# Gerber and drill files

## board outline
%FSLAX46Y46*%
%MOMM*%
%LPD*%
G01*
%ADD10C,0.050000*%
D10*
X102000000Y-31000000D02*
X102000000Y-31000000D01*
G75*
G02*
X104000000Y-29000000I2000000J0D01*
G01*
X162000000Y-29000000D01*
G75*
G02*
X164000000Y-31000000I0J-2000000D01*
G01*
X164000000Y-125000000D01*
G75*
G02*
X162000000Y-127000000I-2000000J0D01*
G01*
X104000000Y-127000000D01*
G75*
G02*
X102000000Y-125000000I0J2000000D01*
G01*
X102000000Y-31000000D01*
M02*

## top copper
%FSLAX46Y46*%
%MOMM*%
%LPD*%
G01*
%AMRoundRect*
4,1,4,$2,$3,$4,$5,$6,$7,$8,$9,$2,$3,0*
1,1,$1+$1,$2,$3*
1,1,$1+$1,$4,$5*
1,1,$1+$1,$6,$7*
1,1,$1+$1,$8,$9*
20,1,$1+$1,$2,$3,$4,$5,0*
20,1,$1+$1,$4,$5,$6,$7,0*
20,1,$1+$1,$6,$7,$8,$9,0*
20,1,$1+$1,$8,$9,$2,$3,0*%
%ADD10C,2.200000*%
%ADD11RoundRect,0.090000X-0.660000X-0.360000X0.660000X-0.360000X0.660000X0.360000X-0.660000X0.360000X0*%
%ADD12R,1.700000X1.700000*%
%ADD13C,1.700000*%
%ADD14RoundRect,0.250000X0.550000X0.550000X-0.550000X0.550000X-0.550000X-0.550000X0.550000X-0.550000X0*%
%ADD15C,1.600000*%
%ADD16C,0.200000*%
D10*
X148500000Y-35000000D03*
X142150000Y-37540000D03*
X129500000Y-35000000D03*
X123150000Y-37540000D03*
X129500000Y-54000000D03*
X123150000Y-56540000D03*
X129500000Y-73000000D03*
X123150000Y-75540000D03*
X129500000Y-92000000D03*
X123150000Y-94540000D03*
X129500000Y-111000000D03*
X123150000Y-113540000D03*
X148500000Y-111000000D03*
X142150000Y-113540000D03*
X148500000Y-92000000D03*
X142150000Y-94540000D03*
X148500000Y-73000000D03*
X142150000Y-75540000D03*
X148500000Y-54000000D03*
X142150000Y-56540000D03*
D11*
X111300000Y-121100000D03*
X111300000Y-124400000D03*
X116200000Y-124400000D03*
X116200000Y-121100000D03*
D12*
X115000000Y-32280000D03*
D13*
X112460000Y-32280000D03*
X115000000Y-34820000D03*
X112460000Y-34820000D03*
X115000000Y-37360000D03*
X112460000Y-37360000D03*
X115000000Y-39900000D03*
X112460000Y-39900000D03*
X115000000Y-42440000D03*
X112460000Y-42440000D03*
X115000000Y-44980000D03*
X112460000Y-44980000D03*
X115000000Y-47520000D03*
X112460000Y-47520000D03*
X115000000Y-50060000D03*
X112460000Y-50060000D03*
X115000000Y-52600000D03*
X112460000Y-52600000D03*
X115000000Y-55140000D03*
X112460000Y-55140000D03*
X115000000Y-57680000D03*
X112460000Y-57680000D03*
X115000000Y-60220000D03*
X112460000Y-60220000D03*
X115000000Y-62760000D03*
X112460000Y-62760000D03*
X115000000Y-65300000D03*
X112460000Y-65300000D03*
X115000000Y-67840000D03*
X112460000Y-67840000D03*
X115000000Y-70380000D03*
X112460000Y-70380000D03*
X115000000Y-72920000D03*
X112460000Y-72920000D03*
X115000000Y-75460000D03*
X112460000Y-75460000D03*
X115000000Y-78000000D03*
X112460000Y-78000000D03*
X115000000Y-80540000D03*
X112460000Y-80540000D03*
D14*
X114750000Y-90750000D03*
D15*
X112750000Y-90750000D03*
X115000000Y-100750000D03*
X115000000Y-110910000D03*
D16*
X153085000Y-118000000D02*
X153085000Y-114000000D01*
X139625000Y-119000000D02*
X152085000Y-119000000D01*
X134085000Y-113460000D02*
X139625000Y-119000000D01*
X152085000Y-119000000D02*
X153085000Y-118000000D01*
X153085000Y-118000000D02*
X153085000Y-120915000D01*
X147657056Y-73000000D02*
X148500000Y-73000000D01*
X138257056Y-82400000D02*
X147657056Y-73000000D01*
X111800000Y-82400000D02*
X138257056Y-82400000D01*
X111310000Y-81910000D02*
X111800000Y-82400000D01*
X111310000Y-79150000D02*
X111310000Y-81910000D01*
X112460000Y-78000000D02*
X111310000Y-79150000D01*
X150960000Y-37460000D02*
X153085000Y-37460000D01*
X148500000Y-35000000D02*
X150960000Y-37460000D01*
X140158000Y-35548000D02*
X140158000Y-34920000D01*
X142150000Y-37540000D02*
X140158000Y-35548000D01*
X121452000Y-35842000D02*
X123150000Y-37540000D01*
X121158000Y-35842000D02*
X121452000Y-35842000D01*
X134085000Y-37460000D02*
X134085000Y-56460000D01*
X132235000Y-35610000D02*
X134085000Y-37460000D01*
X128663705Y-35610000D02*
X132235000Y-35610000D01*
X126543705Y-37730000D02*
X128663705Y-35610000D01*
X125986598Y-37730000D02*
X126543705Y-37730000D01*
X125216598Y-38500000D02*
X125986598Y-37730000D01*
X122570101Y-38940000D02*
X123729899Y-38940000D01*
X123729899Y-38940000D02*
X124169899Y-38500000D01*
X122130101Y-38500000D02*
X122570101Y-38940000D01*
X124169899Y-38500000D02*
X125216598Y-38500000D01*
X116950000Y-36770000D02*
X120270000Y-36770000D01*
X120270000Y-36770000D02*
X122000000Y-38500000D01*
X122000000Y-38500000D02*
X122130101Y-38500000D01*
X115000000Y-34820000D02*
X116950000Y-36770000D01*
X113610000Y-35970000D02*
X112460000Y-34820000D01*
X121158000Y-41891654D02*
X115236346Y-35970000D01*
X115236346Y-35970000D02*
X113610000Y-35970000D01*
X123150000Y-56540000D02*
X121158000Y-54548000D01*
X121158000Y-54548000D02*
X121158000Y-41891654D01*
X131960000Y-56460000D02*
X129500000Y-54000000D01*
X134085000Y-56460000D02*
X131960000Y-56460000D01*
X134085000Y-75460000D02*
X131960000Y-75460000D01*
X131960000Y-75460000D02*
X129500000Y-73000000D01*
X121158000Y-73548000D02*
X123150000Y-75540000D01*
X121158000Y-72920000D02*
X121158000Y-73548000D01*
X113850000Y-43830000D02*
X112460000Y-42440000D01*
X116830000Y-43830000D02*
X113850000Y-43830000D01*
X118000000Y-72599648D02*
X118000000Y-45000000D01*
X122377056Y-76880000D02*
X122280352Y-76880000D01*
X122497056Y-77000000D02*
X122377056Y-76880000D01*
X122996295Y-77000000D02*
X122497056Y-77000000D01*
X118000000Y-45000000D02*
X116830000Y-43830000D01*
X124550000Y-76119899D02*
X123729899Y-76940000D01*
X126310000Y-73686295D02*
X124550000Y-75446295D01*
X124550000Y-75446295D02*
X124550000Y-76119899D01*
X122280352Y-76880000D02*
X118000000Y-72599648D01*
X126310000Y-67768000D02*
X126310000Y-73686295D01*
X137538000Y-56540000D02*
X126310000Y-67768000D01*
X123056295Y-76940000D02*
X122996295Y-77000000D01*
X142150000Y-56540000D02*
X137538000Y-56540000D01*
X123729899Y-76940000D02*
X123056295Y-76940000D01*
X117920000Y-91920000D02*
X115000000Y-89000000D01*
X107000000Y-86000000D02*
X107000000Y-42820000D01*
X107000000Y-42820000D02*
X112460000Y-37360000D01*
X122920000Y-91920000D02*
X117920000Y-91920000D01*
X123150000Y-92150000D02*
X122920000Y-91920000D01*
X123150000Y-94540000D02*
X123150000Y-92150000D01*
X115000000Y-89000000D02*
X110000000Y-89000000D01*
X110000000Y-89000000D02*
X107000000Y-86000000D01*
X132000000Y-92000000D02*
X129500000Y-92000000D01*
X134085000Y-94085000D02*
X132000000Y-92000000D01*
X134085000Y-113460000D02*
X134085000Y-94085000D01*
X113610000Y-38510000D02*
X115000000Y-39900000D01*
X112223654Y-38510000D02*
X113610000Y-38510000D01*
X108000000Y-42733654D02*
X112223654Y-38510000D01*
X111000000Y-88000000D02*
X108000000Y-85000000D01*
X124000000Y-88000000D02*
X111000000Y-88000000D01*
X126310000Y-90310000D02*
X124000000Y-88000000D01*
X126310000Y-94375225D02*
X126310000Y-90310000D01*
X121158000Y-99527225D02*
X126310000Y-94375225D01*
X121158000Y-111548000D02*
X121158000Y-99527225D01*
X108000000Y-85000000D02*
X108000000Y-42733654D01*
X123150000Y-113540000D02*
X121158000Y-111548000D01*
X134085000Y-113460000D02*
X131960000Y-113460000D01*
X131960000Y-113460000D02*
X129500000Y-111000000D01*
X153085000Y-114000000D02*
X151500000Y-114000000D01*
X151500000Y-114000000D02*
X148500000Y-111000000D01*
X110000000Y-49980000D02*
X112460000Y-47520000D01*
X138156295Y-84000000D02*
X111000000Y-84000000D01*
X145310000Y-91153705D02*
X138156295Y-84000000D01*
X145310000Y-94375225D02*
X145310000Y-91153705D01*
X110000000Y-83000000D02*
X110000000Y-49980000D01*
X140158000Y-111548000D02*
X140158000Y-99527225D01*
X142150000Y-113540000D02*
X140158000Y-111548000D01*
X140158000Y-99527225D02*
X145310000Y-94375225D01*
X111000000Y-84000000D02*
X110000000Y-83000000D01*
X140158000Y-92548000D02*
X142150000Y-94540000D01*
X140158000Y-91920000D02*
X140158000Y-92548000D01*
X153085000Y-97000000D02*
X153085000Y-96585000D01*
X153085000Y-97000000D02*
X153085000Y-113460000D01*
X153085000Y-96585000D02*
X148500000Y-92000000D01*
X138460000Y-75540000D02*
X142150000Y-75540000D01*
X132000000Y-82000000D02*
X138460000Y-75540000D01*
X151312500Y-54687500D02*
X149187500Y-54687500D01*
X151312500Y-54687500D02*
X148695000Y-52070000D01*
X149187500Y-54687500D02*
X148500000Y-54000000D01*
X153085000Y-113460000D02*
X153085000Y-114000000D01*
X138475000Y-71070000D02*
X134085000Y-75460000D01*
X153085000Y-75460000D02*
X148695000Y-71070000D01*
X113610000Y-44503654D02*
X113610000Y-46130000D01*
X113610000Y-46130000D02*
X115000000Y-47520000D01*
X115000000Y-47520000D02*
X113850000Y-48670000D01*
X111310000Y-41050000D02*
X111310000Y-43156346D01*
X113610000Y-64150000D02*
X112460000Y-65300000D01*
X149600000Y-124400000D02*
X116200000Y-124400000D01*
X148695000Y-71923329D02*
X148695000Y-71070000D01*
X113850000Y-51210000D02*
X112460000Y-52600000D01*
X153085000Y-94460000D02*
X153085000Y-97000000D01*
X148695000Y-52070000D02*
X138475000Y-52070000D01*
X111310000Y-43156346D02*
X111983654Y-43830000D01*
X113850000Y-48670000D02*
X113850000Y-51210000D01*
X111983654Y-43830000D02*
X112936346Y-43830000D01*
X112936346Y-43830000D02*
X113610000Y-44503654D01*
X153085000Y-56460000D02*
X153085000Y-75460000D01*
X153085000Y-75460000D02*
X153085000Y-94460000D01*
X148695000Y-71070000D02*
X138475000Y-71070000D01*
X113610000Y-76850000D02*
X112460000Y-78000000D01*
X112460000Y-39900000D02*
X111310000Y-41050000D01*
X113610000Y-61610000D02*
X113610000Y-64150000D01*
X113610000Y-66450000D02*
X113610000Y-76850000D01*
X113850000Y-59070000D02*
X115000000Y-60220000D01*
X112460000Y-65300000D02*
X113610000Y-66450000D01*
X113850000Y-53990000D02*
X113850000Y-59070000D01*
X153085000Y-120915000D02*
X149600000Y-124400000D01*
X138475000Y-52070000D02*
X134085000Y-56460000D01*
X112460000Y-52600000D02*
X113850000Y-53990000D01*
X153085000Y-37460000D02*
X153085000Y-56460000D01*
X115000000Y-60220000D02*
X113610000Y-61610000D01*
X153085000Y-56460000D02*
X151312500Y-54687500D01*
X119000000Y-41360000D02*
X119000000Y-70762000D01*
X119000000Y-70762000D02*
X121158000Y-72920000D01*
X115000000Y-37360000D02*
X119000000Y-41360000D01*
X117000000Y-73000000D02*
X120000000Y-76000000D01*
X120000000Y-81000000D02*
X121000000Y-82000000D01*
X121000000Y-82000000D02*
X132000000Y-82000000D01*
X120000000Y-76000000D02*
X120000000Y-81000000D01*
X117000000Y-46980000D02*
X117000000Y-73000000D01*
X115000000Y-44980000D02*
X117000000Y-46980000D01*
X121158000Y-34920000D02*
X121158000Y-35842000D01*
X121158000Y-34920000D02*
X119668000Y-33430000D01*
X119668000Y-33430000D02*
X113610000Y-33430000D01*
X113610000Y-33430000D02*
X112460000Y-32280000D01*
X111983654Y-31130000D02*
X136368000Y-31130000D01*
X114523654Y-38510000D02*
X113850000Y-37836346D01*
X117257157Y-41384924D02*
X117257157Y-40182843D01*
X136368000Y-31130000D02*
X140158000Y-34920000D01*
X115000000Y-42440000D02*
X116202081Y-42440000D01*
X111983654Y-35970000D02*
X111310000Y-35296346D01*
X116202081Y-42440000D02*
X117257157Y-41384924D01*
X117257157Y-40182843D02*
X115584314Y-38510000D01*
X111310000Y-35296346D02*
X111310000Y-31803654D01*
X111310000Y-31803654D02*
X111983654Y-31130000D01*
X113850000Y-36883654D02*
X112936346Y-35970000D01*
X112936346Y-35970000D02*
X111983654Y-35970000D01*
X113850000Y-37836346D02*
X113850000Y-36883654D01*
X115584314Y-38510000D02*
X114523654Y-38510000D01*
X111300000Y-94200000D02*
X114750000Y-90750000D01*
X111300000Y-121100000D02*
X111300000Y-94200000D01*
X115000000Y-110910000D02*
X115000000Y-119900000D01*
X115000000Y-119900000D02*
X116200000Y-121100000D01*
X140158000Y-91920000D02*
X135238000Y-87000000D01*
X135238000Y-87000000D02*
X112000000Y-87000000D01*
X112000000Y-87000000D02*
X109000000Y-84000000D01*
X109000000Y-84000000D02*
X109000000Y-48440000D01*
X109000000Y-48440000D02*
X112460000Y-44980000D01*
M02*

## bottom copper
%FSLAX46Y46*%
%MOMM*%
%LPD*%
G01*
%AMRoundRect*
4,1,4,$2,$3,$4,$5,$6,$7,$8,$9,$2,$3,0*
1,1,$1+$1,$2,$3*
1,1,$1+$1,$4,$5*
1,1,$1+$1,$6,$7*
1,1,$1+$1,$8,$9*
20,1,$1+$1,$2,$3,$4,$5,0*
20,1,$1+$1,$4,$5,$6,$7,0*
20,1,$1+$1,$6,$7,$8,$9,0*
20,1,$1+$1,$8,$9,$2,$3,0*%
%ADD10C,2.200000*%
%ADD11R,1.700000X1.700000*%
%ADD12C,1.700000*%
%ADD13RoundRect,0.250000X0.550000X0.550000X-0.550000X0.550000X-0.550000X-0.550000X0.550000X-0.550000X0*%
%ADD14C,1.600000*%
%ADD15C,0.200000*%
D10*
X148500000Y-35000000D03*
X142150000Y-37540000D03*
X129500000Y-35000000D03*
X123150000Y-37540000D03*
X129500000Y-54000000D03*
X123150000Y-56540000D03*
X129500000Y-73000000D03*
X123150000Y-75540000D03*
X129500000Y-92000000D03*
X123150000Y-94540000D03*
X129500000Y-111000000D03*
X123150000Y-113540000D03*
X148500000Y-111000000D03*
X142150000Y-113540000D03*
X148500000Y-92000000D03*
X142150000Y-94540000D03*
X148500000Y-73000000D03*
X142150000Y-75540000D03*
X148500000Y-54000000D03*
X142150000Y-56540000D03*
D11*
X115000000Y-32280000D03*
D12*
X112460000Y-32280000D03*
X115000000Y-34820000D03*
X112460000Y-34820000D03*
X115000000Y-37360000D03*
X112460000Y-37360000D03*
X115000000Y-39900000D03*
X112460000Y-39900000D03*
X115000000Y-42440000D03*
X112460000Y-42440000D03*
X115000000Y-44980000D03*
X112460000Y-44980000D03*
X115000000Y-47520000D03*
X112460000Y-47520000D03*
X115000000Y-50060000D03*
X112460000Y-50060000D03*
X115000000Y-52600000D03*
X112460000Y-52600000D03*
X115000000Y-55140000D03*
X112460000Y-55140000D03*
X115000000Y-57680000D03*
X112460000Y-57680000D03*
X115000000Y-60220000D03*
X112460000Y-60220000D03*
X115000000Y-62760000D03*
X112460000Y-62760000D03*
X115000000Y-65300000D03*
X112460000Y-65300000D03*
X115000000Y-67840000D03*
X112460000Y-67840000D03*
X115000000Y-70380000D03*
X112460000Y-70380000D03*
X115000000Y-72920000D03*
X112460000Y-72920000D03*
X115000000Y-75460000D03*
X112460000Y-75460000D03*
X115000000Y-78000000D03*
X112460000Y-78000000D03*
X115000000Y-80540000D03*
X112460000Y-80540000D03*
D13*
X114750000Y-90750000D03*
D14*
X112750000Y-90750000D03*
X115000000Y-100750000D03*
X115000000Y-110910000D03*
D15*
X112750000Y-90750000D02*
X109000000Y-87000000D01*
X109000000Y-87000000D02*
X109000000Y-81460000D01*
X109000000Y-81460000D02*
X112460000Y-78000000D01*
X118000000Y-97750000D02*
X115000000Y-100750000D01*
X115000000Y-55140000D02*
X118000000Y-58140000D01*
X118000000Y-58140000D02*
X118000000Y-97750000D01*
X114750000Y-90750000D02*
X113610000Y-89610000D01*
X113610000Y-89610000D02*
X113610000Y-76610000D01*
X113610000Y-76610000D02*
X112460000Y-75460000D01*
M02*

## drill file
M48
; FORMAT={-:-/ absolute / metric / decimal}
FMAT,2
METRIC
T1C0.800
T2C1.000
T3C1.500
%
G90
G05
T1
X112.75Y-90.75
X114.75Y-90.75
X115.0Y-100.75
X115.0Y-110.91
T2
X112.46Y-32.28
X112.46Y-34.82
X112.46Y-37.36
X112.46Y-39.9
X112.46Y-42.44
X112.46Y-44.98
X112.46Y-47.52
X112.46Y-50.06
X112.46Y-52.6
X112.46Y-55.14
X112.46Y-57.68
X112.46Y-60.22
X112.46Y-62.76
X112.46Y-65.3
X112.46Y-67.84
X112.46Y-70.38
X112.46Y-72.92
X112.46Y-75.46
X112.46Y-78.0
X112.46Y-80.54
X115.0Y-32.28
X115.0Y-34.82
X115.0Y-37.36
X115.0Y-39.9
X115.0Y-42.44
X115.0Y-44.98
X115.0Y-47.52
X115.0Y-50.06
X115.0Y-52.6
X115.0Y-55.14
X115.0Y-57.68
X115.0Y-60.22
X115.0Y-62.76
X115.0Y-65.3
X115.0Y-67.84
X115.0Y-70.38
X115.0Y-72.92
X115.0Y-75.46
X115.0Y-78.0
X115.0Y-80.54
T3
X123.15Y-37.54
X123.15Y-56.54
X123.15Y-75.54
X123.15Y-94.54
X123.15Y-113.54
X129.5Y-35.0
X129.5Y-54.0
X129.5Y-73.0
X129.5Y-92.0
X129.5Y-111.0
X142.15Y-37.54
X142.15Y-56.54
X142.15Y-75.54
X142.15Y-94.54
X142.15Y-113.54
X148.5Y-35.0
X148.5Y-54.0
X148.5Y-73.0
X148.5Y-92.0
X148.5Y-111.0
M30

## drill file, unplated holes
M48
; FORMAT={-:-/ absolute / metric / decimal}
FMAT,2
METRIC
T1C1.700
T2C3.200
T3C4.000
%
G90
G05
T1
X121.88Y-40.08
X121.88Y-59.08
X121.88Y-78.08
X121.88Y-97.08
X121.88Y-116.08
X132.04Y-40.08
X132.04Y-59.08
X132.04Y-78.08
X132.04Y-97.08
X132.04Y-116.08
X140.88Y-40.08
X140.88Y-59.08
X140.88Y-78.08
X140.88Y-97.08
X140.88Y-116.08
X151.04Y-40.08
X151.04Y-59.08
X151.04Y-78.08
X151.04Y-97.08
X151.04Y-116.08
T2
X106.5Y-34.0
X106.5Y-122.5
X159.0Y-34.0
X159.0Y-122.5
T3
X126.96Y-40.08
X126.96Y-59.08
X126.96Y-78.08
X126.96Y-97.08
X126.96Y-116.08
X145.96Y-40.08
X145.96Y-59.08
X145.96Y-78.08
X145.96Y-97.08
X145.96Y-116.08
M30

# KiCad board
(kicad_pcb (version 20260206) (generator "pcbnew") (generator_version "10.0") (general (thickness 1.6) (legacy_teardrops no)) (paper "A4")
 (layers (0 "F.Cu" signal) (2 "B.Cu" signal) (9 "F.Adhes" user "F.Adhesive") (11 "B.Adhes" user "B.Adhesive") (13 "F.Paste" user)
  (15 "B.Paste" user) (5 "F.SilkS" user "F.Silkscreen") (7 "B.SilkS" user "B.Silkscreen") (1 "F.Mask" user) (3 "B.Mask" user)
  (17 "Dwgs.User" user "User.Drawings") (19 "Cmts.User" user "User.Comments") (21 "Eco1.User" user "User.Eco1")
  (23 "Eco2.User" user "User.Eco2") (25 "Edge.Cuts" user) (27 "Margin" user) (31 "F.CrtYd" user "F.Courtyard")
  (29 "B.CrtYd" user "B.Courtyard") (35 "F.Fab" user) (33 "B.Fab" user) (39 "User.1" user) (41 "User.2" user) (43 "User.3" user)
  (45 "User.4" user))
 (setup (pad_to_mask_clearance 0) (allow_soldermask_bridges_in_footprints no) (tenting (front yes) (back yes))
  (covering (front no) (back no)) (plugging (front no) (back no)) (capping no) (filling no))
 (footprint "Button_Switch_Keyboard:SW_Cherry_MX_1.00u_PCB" (layer "F.Cu") (at 148.5 35)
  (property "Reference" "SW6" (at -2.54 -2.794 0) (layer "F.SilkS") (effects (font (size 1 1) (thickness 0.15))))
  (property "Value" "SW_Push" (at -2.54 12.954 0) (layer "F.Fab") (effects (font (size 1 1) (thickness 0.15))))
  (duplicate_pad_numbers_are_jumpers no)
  (pad "" np_thru_hole circle (at -7.62 5.08) (size 1.7 1.7) (drill 1.7) (layers "*.Cu" "*.Mask"))
  (pad "" np_thru_hole circle (at -2.54 5.08) (size 4 4) (drill 4) (layers "*.Cu" "*.Mask"))
  (pad "" np_thru_hole circle (at 2.54 5.08) (size 1.7 1.7) (drill 1.7) (layers "*.Cu" "*.Mask"))
  (pad "1" thru_hole circle (at 0 0) (size 2.2 2.2) (drill 1.5) (layers "*.Cu" "*.Mask") (remove_unused_layers no) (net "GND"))
  (pad "2" thru_hole circle (at -6.35 2.54) (size 2.2 2.2) (drill 1.5) (layers "*.Cu" "*.Mask") (remove_unused_layers no)
   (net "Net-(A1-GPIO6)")))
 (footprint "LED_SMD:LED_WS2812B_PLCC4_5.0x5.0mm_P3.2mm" (layer "F.Cu") (at 113.75 122.75)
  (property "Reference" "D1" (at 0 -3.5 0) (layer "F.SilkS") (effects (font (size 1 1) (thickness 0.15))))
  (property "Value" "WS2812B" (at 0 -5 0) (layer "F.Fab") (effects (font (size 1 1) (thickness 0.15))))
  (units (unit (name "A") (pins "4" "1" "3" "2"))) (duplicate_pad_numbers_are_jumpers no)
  (pad "1" smd roundrect (at -2.45 -1.65) (size 1.5 0.9) (layers "F.Cu" "F.Mask" "F.Paste") (roundrect_rratio 0.1) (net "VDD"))
  (pad "2" smd roundrect (at -2.45 1.65) (size 1.5 0.9) (layers "F.Cu" "F.Mask" "F.Paste") (roundrect_rratio 0.1)
   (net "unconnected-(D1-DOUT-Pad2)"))
  (pad "3" smd roundrect (at 2.45 1.65) (size 1.5 0.9) (layers "F.Cu" "F.Mask" "F.Paste") (roundrect_rratio 0.1) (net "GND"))
  (pad "4" smd roundrect (at 2.45 -1.65) (size 1.5 0.9) (layers "F.Cu" "F.Mask" "F.Paste") (roundrect_rratio 0.1) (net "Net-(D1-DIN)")))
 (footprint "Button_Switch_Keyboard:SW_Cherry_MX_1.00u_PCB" (layer "F.Cu") (at 129.5 73)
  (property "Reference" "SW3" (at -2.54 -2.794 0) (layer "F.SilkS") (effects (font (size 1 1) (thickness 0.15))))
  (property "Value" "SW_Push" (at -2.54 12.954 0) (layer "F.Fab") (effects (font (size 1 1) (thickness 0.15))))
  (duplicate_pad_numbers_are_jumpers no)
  (pad "" np_thru_hole circle (at -7.62 5.08) (size 1.7 1.7) (drill 1.7) (layers "*.Cu" "*.Mask"))
  (pad "" np_thru_hole circle (at -2.54 5.08) (size 4 4) (drill 4) (layers "*.Cu" "*.Mask"))
  (pad "" np_thru_hole circle (at 2.54 5.08) (size 1.7 1.7) (drill 1.7) (layers "*.Cu" "*.Mask"))
  (pad "1" thru_hole circle (at 0 0) (size 2.2 2.2) (drill 1.5) (layers "*.Cu" "*.Mask") (remove_unused_layers no) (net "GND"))
  (pad "2" thru_hole circle (at -6.35 2.54) (size 2.2 2.2) (drill 1.5) (layers "*.Cu" "*.Mask") (remove_unused_layers no)
   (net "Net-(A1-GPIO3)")))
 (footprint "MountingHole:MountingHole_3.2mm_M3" (layer "F.Cu") (at 159 34)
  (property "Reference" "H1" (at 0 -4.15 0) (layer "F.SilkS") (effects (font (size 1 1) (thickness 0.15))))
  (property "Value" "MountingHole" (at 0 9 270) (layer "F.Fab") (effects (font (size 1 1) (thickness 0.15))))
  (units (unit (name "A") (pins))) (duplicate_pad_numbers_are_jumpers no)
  (pad "" np_thru_hole circle (at 0 0) (size 3.2 3.2) (drill 3.2) (layers "*.Cu" "*.Mask")))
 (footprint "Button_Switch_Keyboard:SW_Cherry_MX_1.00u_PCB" (layer "F.Cu") (at 129.5 35)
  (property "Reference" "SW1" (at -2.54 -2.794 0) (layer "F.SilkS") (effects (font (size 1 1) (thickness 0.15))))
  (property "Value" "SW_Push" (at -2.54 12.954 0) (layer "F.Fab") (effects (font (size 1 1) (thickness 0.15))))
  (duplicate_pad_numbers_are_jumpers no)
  (pad "" np_thru_hole circle (at -7.62 5.08) (size 1.7 1.7) (drill 1.7) (layers "*.Cu" "*.Mask"))
  (pad "" np_thru_hole circle (at -2.54 5.08) (size 4 4) (drill 4) (layers "*.Cu" "*.Mask"))
  (pad "" np_thru_hole circle (at 2.54 5.08) (size 1.7 1.7) (drill 1.7) (layers "*.Cu" "*.Mask"))
  (pad "1" thru_hole circle (at 0 0) (size 2.2 2.2) (drill 1.5) (layers "*.Cu" "*.Mask") (remove_unused_layers no) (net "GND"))
  (pad "2" thru_hole circle (at -6.35 2.54) (size 2.2 2.2) (drill 1.5) (layers "*.Cu" "*.Mask") (remove_unused_layers no)
   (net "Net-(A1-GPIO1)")))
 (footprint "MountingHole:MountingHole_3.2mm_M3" (layer "F.Cu") (at 159 122.5)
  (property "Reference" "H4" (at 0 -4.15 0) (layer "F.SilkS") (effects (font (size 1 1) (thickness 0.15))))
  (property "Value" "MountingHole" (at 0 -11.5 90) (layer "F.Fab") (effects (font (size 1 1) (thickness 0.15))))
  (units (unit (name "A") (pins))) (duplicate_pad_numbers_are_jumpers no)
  (pad "" np_thru_hole circle (at 0 0) (size 3.2 3.2) (drill 3.2) (layers "*.Cu" "*.Mask")))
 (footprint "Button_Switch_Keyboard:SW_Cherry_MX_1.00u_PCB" (layer "F.Cu") (at 148.5 92)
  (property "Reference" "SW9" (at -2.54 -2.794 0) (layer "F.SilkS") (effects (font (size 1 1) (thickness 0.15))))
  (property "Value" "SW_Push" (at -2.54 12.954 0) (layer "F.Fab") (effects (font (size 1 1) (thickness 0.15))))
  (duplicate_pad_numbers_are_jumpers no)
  (pad "" np_thru_hole circle (at -7.62 5.08) (size 1.7 1.7) (drill 1.7) (layers "*.Cu" "*.Mask"))
  (pad "" np_thru_hole circle (at -2.54 5.08) (size 4 4) (drill 4) (layers "*.Cu" "*.Mask"))
  (pad "" np_thru_hole circle (at 2.54 5.08) (size 1.7 1.7) (drill 1.7) (layers "*.Cu" "*.Mask"))
  (pad "1" thru_hole circle (at 0 0) (size 2.2 2.2) (drill 1.5) (layers "*.Cu" "*.Mask") (remove_unused_layers no) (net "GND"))
  (pad "2" thru_hole circle (at -6.35 2.54) (size 2.2 2.2) (drill 1.5) (layers "*.Cu" "*.Mask") (remove_unused_layers no)
   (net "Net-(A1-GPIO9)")))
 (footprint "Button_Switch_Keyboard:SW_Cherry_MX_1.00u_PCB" (layer "F.Cu") (at 148.5 54)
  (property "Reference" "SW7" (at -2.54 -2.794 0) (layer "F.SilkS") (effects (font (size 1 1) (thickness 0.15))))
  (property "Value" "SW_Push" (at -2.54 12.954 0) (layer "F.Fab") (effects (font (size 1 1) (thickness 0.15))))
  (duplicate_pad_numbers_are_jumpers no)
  (pad "" np_thru_hole circle (at -7.62 5.08) (size 1.7 1.7) (drill 1.7) (layers "*.Cu" "*.Mask"))
  (pad "" np_thru_hole circle (at -2.54 5.08) (size 4 4) (drill 4) (layers "*.Cu" "*.Mask"))
  (pad "" np_thru_hole circle (at 2.54 5.08) (size 1.7 1.7) (drill 1.7) (layers "*.Cu" "*.Mask"))
  (pad "1" thru_hole circle (at 0 0) (size 2.2 2.2) (drill 1.5) (layers "*.Cu" "*.Mask") (remove_unused_layers no) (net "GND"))
  (pad "2" thru_hole circle (at -6.35 2.54) (size 2.2 2.2) (drill 1.5) (layers "*.Cu" "*.Mask") (remove_unused_layers no)
   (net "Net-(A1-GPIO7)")))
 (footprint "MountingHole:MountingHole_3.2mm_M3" (layer "F.Cu") (at 106.5 34)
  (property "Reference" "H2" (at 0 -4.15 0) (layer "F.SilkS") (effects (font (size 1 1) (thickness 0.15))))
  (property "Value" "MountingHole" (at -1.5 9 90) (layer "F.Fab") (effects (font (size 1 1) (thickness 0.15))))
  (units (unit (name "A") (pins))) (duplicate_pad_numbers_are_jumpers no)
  (pad "" np_thru_hole circle (at 0 0) (size 3.2 3.2) (drill 3.2) (layers "*.Cu" "*.Mask")))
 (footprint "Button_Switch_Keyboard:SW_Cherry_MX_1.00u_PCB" (layer "F.Cu") (at 148.5 111)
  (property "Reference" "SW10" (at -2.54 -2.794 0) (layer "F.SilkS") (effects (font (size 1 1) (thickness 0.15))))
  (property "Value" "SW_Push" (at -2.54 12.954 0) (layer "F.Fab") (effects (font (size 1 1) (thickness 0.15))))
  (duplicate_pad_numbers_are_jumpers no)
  (pad "" np_thru_hole circle (at -7.62 5.08) (size 1.7 1.7) (drill 1.7) (layers "*.Cu" "*.Mask"))
  (pad "" np_thru_hole circle (at -2.54 5.08) (size 4 4) (drill 4) (layers "*.Cu" "*.Mask"))
  (pad "" np_thru_hole circle (at 2.54 5.08) (size 1.7 1.7) (drill 1.7) (layers "*.Cu" "*.Mask"))
  (pad "1" thru_hole circle (at 0 0) (size 2.2 2.2) (drill 1.5) (layers "*.Cu" "*.Mask") (remove_unused_layers no) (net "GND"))
  (pad "2" thru_hole circle (at -6.35 2.54) (size 2.2 2.2) (drill 1.5) (layers "*.Cu" "*.Mask") (remove_unused_layers no)
   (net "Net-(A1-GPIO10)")))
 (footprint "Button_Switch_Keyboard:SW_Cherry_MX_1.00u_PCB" (layer "F.Cu") (at 148.5 73)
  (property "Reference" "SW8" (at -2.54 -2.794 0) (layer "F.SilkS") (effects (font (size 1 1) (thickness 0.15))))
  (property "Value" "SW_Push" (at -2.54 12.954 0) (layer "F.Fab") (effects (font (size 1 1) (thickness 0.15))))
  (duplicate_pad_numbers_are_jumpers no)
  (pad "" np_thru_hole circle (at -7.62 5.08) (size 1.7 1.7) (drill 1.7) (layers "*.Cu" "*.Mask"))
  (pad "" np_thru_hole circle (at -2.54 5.08) (size 4 4) (drill 4) (layers "*.Cu" "*.Mask"))
  (pad "" np_thru_hole circle (at 2.54 5.08) (size 1.7 1.7) (drill 1.7) (layers "*.Cu" "*.Mask"))
  (pad "1" thru_hole circle (at 0 0) (size 2.2 2.2) (drill 1.5) (layers "*.Cu" "*.Mask") (remove_unused_layers no) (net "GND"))
  (pad "2" thru_hole circle (at -6.35 2.54) (size 2.2 2.2) (drill 1.5) (layers "*.Cu" "*.Mask") (remove_unused_layers no)
   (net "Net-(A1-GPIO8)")))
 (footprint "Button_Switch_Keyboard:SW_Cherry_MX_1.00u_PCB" (layer "F.Cu") (at 129.5 54)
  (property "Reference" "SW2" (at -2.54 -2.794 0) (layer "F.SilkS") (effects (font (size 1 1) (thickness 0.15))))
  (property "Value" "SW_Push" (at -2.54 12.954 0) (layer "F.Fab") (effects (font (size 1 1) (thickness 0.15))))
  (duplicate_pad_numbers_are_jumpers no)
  (pad "" np_thru_hole circle (at -7.62 5.08) (size 1.7 1.7) (drill 1.7) (layers "*.Cu" "*.Mask"))
  (pad "" np_thru_hole circle (at -2.54 5.08) (size 4 4) (drill 4) (layers "*.Cu" "*.Mask"))
  (pad "" np_thru_hole circle (at 2.54 5.08) (size 1.7 1.7) (drill 1.7) (layers "*.Cu" "*.Mask"))
  (pad "1" thru_hole circle (at 0 0) (size 2.2 2.2) (drill 1.5) (layers "*.Cu" "*.Mask") (remove_unused_layers no) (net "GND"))
  (pad "2" thru_hole circle (at -6.35 2.54) (size 2.2 2.2) (drill 1.5) (layers "*.Cu" "*.Mask") (remove_unused_layers no)
   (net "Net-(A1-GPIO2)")))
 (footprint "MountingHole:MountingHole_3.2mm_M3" (layer "F.Cu") (at 106.5 122.5)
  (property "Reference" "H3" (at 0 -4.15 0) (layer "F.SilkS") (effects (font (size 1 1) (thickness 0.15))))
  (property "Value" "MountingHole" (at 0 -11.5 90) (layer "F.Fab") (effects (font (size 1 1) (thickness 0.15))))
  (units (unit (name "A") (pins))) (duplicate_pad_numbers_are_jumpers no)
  (pad "" np_thru_hole circle (at 0 0) (size 3.2 3.2) (drill 3.2) (layers "*.Cu" "*.Mask")))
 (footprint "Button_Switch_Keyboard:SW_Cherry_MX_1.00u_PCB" (layer "F.Cu") (at 129.5 111)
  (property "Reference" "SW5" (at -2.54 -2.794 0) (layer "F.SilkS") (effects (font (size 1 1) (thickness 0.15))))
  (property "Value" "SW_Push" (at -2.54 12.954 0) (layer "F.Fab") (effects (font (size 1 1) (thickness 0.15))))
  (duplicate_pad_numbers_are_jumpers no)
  (pad "" np_thru_hole circle (at -7.62 5.08) (size 1.7 1.7) (drill 1.7) (layers "*.Cu" "*.Mask"))
  (pad "" np_thru_hole circle (at -2.54 5.08) (size 4 4) (drill 4) (layers "*.Cu" "*.Mask"))
  (pad "" np_thru_hole circle (at 2.54 5.08) (size 1.7 1.7) (drill 1.7) (layers "*.Cu" "*.Mask"))
  (pad "1" thru_hole circle (at 0 0) (size 2.2 2.2) (drill 1.5) (layers "*.Cu" "*.Mask") (remove_unused_layers no) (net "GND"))
  (pad "2" thru_hole circle (at -6.35 2.54) (size 2.2 2.2) (drill 1.5) (layers "*.Cu" "*.Mask") (remove_unused_layers no)
   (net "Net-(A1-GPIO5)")))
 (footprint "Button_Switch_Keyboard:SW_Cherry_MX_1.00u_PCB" (layer "F.Cu") (at 129.5 92)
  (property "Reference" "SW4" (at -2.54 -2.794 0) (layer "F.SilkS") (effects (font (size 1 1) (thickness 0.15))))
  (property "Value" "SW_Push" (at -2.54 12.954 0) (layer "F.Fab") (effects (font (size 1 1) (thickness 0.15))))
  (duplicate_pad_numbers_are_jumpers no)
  (pad "" np_thru_hole circle (at -7.62 5.08) (size 1.7 1.7) (drill 1.7) (layers "*.Cu" "*.Mask"))
  (pad "" np_thru_hole circle (at -2.54 5.08) (size 4 4) (drill 4) (layers "*.Cu" "*.Mask"))
  (pad "" np_thru_hole circle (at 2.54 5.08) (size 1.7 1.7) (drill 1.7) (layers "*.Cu" "*.Mask"))
  (pad "1" thru_hole circle (at 0 0) (size 2.2 2.2) (drill 1.5) (layers "*.Cu" "*.Mask") (remove_unused_layers no) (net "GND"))
  (pad "2" thru_hole circle (at -6.35 2.54) (size 2.2 2.2) (drill 1.5) (layers "*.Cu" "*.Mask") (remove_unused_layers no)
   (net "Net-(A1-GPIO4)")))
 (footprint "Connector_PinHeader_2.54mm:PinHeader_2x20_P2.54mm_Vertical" (layer "B.Cu") (at 115 32.28 180)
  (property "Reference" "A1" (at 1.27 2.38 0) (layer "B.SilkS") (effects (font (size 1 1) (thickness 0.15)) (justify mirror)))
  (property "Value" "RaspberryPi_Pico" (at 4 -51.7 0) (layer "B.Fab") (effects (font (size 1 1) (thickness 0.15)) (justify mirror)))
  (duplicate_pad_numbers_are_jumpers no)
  (pad "1" thru_hole rect (at 0 0 180) (size 1.7 1.7) (drill 1) (layers "*.Cu" "*.Mask") (remove_unused_layers no)
   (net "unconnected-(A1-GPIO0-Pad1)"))
  (pad "2" thru_hole circle (at 2.54 0 180) (size 1.7 1.7) (drill 1) (layers "*.Cu" "*.Mask") (remove_unused_layers no)
   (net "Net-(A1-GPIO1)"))
  (pad "3" thru_hole circle (at 0 -2.54 180) (size 1.7 1.7) (drill 1) (layers "*.Cu" "*.Mask") (remove_unused_layers no) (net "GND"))
  (pad "4" thru_hole circle (at 2.54 -2.54 180) (size 1.7 1.7) (drill 1) (layers "*.Cu" "*.Mask") (remove_unused_layers no)
   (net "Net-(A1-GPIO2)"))
  (pad "5" thru_hole circle (at 0 -5.08 180) (size 1.7 1.7) (drill 1) (layers "*.Cu" "*.Mask") (remove_unused_layers no)
   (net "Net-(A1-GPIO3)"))
  (pad "6" thru_hole circle (at 2.54 -5.08 180) (size 1.7 1.7) (drill 1) (layers "*.Cu" "*.Mask") (remove_unused_layers no)
   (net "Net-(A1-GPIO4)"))
  (pad "7" thru_hole circle (at 0 -7.62 180) (size 1.7 1.7) (drill 1) (layers "*.Cu" "*.Mask") (remove_unused_layers no)
   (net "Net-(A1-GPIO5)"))
  (pad "8" thru_hole circle (at 2.54 -7.62 180) (size 1.7 1.7) (drill 1) (layers "*.Cu" "*.Mask") (remove_unused_layers no) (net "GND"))
  (pad "9" thru_hole circle (at 0 -10.16 180) (size 1.7 1.7) (drill 1) (layers "*.Cu" "*.Mask") (remove_unused_layers no)
   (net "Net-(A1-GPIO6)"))
  (pad "10" thru_hole circle (at 2.54 -10.16 180) (size 1.7 1.7) (drill 1) (layers "*.Cu" "*.Mask") (remove_unused_layers no)
   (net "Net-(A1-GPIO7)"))
  (pad "11" thru_hole circle (at 0 -12.7 180) (size 1.7 1.7) (drill 1) (layers "*.Cu" "*.Mask") (remove_unused_layers no)
   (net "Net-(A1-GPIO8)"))
  (pad "12" thru_hole circle (at 2.54 -12.7 180) (size 1.7 1.7) (drill 1) (layers "*.Cu" "*.Mask") (remove_unused_layers no)
   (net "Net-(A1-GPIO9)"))
  (pad "13" thru_hole circle (at 0 -15.24 180) (size 1.7 1.7) (drill 1) (layers "*.Cu" "*.Mask") (remove_unused_layers no) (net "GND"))
  (pad "14" thru_hole circle (at 2.54 -15.24 180) (size 1.7 1.7) (drill 1) (layers "*.Cu" "*.Mask") (remove_unused_layers no)
   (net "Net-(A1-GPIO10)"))
  (pad "15" thru_hole circle (at 0 -17.78 180) (size 1.7 1.7) (drill 1) (layers "*.Cu" "*.Mask") (remove_unused_layers no)
   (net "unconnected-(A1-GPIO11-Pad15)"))
  (pad "16" thru_hole circle (at 2.54 -17.78 180) (size 1.7 1.7) (drill 1) (layers "*.Cu" "*.Mask") (remove_unused_layers no)
   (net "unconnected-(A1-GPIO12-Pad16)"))
  (pad "17" thru_hole circle (at 0 -20.32 180) (size 1.7 1.7) (drill 1) (layers "*.Cu" "*.Mask") (remove_unused_layers no)
   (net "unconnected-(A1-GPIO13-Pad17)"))
  (pad "18" thru_hole circle (at 2.54 -20.32 180) (size 1.7 1.7) (drill 1) (layers "*.Cu" "*.Mask") (remove_unused_layers no) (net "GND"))
  (pad "19" thru_hole circle (at 0 -22.86 180) (size 1.7 1.7) (drill 1) (layers "*.Cu" "*.Mask") (remove_unused_layers no)
   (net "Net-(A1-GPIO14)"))
  (pad "20" thru_hole circle (at 2.54 -22.86 180) (size 1.7 1.7) (drill 1) (layers "*.Cu" "*.Mask") (remove_unused_layers no)
   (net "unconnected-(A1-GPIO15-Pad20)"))
  (pad "21" thru_hole circle (at 0 -25.4 180) (size 1.7 1.7) (drill 1) (layers "*.Cu" "*.Mask") (remove_unused_layers no)
   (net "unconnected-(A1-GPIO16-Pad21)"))
  (pad "22" thru_hole circle (at 2.54 -25.4 180) (size 1.7 1.7) (drill 1) (layers "*.Cu" "*.Mask") (remove_unused_layers no)
   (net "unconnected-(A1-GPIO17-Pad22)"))
  (pad "23" thru_hole circle (at 0 -27.94 180) (size 1.7 1.7) (drill 1) (layers "*.Cu" "*.Mask") (remove_unused_layers no) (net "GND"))
  (pad "24" thru_hole circle (at 2.54 -27.94 180) (size 1.7 1.7) (drill 1) (layers "*.Cu" "*.Mask") (remove_unused_layers no)
   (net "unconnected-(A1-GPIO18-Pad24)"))
  (pad "25" thru_hole circle (at 0 -30.48 180) (size 1.7 1.7) (drill 1) (layers "*.Cu" "*.Mask") (remove_unused_layers no)
   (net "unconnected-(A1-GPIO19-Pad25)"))
  (pad "26" thru_hole circle (at 2.54 -30.48 180) (size 1.7 1.7) (drill 1) (layers "*.Cu" "*.Mask") (remove_unused_layers no)
   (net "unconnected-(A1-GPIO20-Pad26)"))
  (pad "27" thru_hole circle (at 0 -33.02 180) (size 1.7 1.7) (drill 1) (layers "*.Cu" "*.Mask") (remove_unused_layers no)
   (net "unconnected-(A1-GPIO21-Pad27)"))
  (pad "28" thru_hole circle (at 2.54 -33.02 180) (size 1.7 1.7) (drill 1) (layers "*.Cu" "*.Mask") (remove_unused_layers no) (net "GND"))
  (pad "29" thru_hole circle (at 0 -35.56 180) (size 1.7 1.7) (drill 1) (layers "*.Cu" "*.Mask") (remove_unused_layers no)
   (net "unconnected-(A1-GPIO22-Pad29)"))
  (pad "30" thru_hole circle (at 2.54 -35.56 180) (size 1.7 1.7) (drill 1) (layers "*.Cu" "*.Mask") (remove_unused_layers no)
   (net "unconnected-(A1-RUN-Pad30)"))
  (pad "31" thru_hole circle (at 0 -38.1 180) (size 1.7 1.7) (drill 1) (layers "*.Cu" "*.Mask") (remove_unused_layers no)
   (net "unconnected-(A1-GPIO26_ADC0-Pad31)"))
  (pad "32" thru_hole circle (at 2.54 -38.1 180) (size 1.7 1.7) (drill 1) (layers "*.Cu" "*.Mask") (remove_unused_layers no)
   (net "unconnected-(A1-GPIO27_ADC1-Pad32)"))
  (pad "33" thru_hole circle (at 0 -40.64 180) (size 1.7 1.7) (drill 1) (layers "*.Cu" "*.Mask") (remove_unused_layers no)
   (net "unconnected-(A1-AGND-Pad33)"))
  (pad "34" thru_hole circle (at 2.54 -40.64 180) (size 1.7 1.7) (drill 1) (layers "*.Cu" "*.Mask") (remove_unused_layers no)
   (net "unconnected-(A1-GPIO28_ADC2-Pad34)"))
  (pad "35" thru_hole circle (at 0 -43.18 180) (size 1.7 1.7) (drill 1) (layers "*.Cu" "*.Mask") (remove_unused_layers no)
   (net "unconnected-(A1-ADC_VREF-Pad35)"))
  (pad "36" thru_hole circle (at 2.54 -43.18 180) (size 1.7 1.7) (drill 1) (layers "*.Cu" "*.Mask") (remove_unused_layers no) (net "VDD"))
  (pad "37" thru_hole circle (at 0 -45.72 180) (size 1.7 1.7) (drill 1) (layers "*.Cu" "*.Mask") (remove_unused_layers no)
   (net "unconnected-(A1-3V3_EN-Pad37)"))
  (pad "38" thru_hole circle (at 2.54 -45.72 180) (size 1.7 1.7) (drill 1) (layers "*.Cu" "*.Mask") (remove_unused_layers no) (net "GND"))
  (pad "39" thru_hole circle (at 0 -48.26 180) (size 1.7 1.7) (drill 1) (layers "*.Cu" "*.Mask") (remove_unused_layers no)
   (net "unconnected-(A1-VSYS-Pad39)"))
  (pad "40" thru_hole circle (at 2.54 -48.26 180) (size 1.7 1.7) (drill 1) (layers "*.Cu" "*.Mask") (remove_unused_layers no)
   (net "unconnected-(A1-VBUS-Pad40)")))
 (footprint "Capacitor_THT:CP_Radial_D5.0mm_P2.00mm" (layer "B.Cu") (at 114.75 90.75 180)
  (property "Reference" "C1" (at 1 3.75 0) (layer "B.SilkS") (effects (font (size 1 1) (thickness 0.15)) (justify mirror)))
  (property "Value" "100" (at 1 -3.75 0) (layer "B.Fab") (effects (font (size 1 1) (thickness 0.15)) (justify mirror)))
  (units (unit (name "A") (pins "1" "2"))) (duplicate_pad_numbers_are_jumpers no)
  (pad "1" thru_hole roundrect (at 0 0 180) (size 1.6 1.6) (drill 0.8) (layers "*.Cu" "*.Mask") (remove_unused_layers no)
   (roundrect_rratio 0.15625) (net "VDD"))
  (pad "2" thru_hole circle (at 2 0 180) (size 1.6 1.6) (drill 0.8) (layers "*.Cu" "*.Mask") (remove_unused_layers no) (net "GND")))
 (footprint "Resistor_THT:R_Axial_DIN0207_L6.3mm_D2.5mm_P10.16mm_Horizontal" (layer "B.Cu") (at 115 100.75 -90)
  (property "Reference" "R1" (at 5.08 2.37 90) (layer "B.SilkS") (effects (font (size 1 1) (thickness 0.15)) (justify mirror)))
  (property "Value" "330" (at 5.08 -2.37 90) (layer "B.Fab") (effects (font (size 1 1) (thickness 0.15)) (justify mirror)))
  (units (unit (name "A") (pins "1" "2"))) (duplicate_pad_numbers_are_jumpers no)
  (pad "1" thru_hole circle (at 0 0 270) (size 1.6 1.6) (drill 0.8) (layers "*.Cu" "*.Mask") (remove_unused_layers no)
   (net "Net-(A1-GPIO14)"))
  (pad "2" thru_hole circle (at 10.16 0 270) (size 1.6 1.6) (drill 0.8) (layers "*.Cu" "*.Mask") (remove_unused_layers no)
   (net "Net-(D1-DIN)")))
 (gr_rect (start 102 29) (end 164 127) (radius 2) (stroke (width 0.05) (type solid)) (fill no) (layer "Edge.Cuts"))
 (segment (start 153.085 118) (end 153.085 120.915) (width 0.2) (layer "F.Cu") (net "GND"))
 (segment (start 134.085 113.46) (end 134.085 94.085) (width 0.2) (layer "F.Cu") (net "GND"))
 (segment (start 153.085 114) (end 151.5 114) (width 0.2) (layer "F.Cu") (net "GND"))
 (segment (start 153.085 113.46) (end 153.085 114) (width 0.2) (layer "F.Cu") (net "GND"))
 (segment (start 138.475 71.07) (end 134.085 75.46) (width 0.2) (layer "F.Cu") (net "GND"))
 (segment (start 153.085 75.46) (end 148.695 71.07) (width 0.2) (layer "F.Cu") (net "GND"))
 (segment (start 113.61 44.503654) (end 113.61 46.13) (width 0.2) (layer "F.Cu") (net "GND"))
 (segment (start 149.1875 54.6875) (end 148.5 54) (width 0.2) (layer "F.Cu") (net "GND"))
 (segment (start 131.96 56.46) (end 129.5 54) (width 0.2) (layer "F.Cu") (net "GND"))
 (segment (start 134.085 113.46) (end 139.625 119) (width 0.2) (layer "F.Cu") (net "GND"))
 (segment (start 113.61 46.13) (end 115 47.52) (width 0.2) (layer "F.Cu") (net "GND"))
 (segment (start 128.663705 35.61) (end 132.235 35.61) (width 0.2) (layer "F.Cu") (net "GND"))
 (segment (start 112.46 78) (end 111.31 79.15) (width 0.2) (layer "F.Cu") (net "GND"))
 (segment (start 115 47.52) (end 113.85 48.67) (width 0.2) (layer "F.Cu") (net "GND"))
 (segment (start 153.085 118) (end 153.085 114) (width 0.2) (layer "F.Cu") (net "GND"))
 (segment (start 111.31 41.05) (end 111.31 43.156346) (width 0.2) (layer "F.Cu") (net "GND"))
 (segment (start 153.085 96.585) (end 148.5 92) (width 0.2) (layer "F.Cu") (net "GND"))
 (segment (start 113.61 64.15) (end 112.46 65.3) (width 0.2) (layer "F.Cu") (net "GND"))
 (segment (start 149.6 124.4) (end 116.2 124.4) (width 0.2) (layer "F.Cu") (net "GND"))
 (segment (start 148.695 71.923329) (end 148.695 71.07) (width 0.2) (layer "F.Cu") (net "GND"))
 (segment (start 148.5 35) (end 150.96 37.46) (width 0.2) (layer "F.Cu") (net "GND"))
 (segment (start 134.085 113.46) (end 131.96 113.46) (width 0.2) (layer "F.Cu") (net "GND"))
 (segment (start 113.85 51.21) (end 112.46 52.6) (width 0.2) (layer "F.Cu") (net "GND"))
 (segment (start 116.95 36.77) (end 120.27 36.77) (width 0.2) (layer "F.Cu") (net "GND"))
 (segment (start 123.729899 38.94) (end 124.169899 38.5) (width 0.2) (layer "F.Cu") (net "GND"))
 (segment (start 153.085 94.46) (end 153.085 97) (width 0.2) (layer "F.Cu") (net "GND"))
 (segment (start 148.695 52.07) (end 138.475 52.07) (width 0.2) (layer "F.Cu") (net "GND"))
 (segment (start 150.96 37.46) (end 153.085 37.46) (width 0.2) (layer "F.Cu") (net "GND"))
 (segment (start 122.570101 38.94) (end 123.729899 38.94) (width 0.2) (layer "F.Cu") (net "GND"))
 (segment (start 111.31 43.156346) (end 111.983654 43.83) (width 0.2) (layer "F.Cu") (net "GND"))
 (segment (start 151.3125 54.6875) (end 148.695 52.07) (width 0.2) (layer "F.Cu") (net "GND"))
 (segment (start 134.085 56.46) (end 131.96 56.46) (width 0.2) (layer "F.Cu") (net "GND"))
 (segment (start 134.085 75.46) (end 131.96 75.46) (width 0.2) (layer "F.Cu") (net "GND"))
 (segment (start 120.27 36.77) (end 122 38.5) (width 0.2) (layer "F.Cu") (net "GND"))
 (segment (start 125.216598 38.5) (end 125.986598 37.73) (width 0.2) (layer "F.Cu") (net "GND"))
 (segment (start 125.986598 37.73) (end 126.543705 37.73) (width 0.2) (layer "F.Cu") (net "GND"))
 (segment (start 111.31 81.91) (end 111.8 82.4) (width 0.2) (layer "F.Cu") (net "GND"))
 (segment (start 131.96 75.46) (end 129.5 73) (width 0.2) (layer "F.Cu") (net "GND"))
 (segment (start 113.85 48.67) (end 113.85 51.21) (width 0.2) (layer "F.Cu") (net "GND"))
 (segment (start 126.543705 37.73) (end 128.663705 35.61) (width 0.2) (layer "F.Cu") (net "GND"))
 (segment (start 131.96 113.46) (end 129.5 111) (width 0.2) (layer "F.Cu") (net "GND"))
 (segment (start 111.983654 43.83) (end 112.936346 43.83) (width 0.2) (layer "F.Cu") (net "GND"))
 (segment (start 147.657056 73) (end 148.5 73) (width 0.2) (layer "F.Cu") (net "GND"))
 (segment (start 112.936346 43.83) (end 113.61 44.503654) (width 0.2) (layer "F.Cu") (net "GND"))
 (segment (start 153.085 56.46) (end 153.085 75.46) (width 0.2) (layer "F.Cu") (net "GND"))
 (segment (start 132.235 35.61) (end 134.085 37.46) (width 0.2) (layer "F.Cu") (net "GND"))
 (segment (start 153.085 97) (end 153.085 113.46) (width 0.2) (layer "F.Cu") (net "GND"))
 (segment (start 134.085 94.085) (end 132 92) (width 0.2) (layer "F.Cu") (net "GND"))
 (segment (start 124.169899 38.5) (end 125.216598 38.5) (width 0.2) (layer "F.Cu") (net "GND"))
 (segment (start 153.085 97) (end 153.085 96.585) (width 0.2) (layer "F.Cu") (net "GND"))
 (segment (start 153.085 75.46) (end 153.085 94.46) (width 0.2) (layer "F.Cu") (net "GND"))
 (segment (start 122.130101 38.5) (end 122.570101 38.94) (width 0.2) (layer "F.Cu") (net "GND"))
 (segment (start 122 38.5) (end 122.130101 38.5) (width 0.2) (layer "F.Cu") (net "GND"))
 (segment (start 111.8 82.4) (end 138.257056 82.4) (width 0.2) (layer "F.Cu") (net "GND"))
 (segment (start 148.695 71.07) (end 138.475 71.07) (width 0.2) (layer "F.Cu") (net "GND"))
 (segment (start 115 34.82) (end 116.95 36.77) (width 0.2) (layer "F.Cu") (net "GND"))
 (segment (start 152.085 119) (end 153.085 118) (width 0.2) (layer "F.Cu") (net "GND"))
 (segment (start 113.61 76.85) (end 112.46 78) (width 0.2) (layer "F.Cu") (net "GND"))
 (segment (start 112.46 39.9) (end 111.31 41.05) (width 0.2) (layer "F.Cu") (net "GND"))
 (segment (start 138.257056 82.4) (end 147.657056 73) (width 0.2) (layer "F.Cu") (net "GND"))
 (segment (start 113.61 61.61) (end 113.61 64.15) (width 0.2) (layer "F.Cu") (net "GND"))
 (segment (start 113.61 66.45) (end 113.61 76.85) (width 0.2) (layer "F.Cu") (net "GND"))
 (segment (start 113.85 59.07) (end 115 60.22) (width 0.2) (layer "F.Cu") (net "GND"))
 (segment (start 112.46 65.3) (end 113.61 66.45) (width 0.2) (layer "F.Cu") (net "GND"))
 (segment (start 111.31 79.15) (end 111.31 81.91) (width 0.2) (layer "F.Cu") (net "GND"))
 (segment (start 113.85 53.99) (end 113.85 59.07) (width 0.2) (layer "F.Cu") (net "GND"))
 (segment (start 153.085 120.915) (end 149.6 124.4) (width 0.2) (layer "F.Cu") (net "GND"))
 (segment (start 138.475 52.07) (end 134.085 56.46) (width 0.2) (layer "F.Cu") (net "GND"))
 (segment (start 112.46 52.6) (end 113.85 53.99) (width 0.2) (layer "F.Cu") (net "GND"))
 (segment (start 153.085 37.46) (end 153.085 56.46) (width 0.2) (layer "F.Cu") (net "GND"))
 (segment (start 115 60.22) (end 113.61 61.61) (width 0.2) (layer "F.Cu") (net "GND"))
 (segment (start 134.085 37.46) (end 134.085 56.46) (width 0.2) (layer "F.Cu") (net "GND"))
 (segment (start 132 92) (end 129.5 92) (width 0.2) (layer "F.Cu") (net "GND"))
 (segment (start 153.085 56.46) (end 151.3125 54.6875) (width 0.2) (layer "F.Cu") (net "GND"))
 (segment (start 139.625 119) (end 152.085 119) (width 0.2) (layer "F.Cu") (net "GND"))
 (segment (start 151.3125 54.6875) (end 149.1875 54.6875) (width 0.2) (layer "F.Cu") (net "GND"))
 (segment (start 151.5 114) (end 148.5 111) (width 0.2) (layer "F.Cu") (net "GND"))
 (segment (start 112.75 90.75) (end 109 87) (width 0.2) (layer "B.Cu") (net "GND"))
 (segment (start 109 87) (end 109 81.46) (width 0.2) (layer "B.Cu") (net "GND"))
 (segment (start 109 81.46) (end 112.46 78) (width 0.2) (layer "B.Cu") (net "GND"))
 (segment (start 142.15 37.54) (end 140.158 35.548) (width 0.2) (layer "F.Cu") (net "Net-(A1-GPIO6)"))
 (segment (start 111.983654 31.13) (end 136.368 31.13) (width 0.2) (layer "F.Cu") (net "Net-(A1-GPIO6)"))
 (segment (start 114.523654 38.51) (end 113.85 37.836346) (width 0.2) (layer "F.Cu") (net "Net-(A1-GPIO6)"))
 (segment (start 117.257157 41.384924) (end 117.257157 40.182843) (width 0.2) (layer "F.Cu") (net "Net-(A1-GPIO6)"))
 (segment (start 136.368 31.13) (end 140.158 34.92) (width 0.2) (layer "F.Cu") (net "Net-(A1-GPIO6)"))
 (segment (start 115 42.44) (end 116.202081 42.44) (width 0.2) (layer "F.Cu") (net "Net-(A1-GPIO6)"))
 (segment (start 111.983654 35.97) (end 111.31 35.296346) (width 0.2) (layer "F.Cu") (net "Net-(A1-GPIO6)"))
 (segment (start 116.202081 42.44) (end 117.257157 41.384924) (width 0.2) (layer "F.Cu") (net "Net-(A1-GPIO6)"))
 (segment (start 117.257157 40.182843) (end 115.584314 38.51) (width 0.2) (layer "F.Cu") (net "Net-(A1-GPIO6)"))
 (segment (start 111.31 35.296346) (end 111.31 31.803654) (width 0.2) (layer "F.Cu") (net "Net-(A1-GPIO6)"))
 (segment (start 111.31 31.803654) (end 111.983654 31.13) (width 0.2) (layer "F.Cu") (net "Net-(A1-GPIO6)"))
 (segment (start 113.85 36.883654) (end 112.936346 35.97) (width 0.2) (layer "F.Cu") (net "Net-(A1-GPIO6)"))
 (segment (start 112.936346 35.97) (end 111.983654 35.97) (width 0.2) (layer "F.Cu") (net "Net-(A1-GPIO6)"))
 (segment (start 113.85 37.836346) (end 113.85 36.883654) (width 0.2) (layer "F.Cu") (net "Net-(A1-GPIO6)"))
 (segment (start 140.158 35.548) (end 140.158 34.92) (width 0.2) (layer "F.Cu") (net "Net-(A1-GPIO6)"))
 (segment (start 115.584314 38.51) (end 114.523654 38.51) (width 0.2) (layer "F.Cu") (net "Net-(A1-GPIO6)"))
 (segment (start 111.3 94.2) (end 114.75 90.75) (width 0.2) (layer "F.Cu") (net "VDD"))
 (segment (start 111.3 121.1) (end 111.3 94.2) (width 0.2) (layer "F.Cu") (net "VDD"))
 (segment (start 114.75 90.75) (end 113.61 89.61) (width 0.2) (layer "B.Cu") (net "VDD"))
 (segment (start 113.61 89.61) (end 113.61 76.61) (width 0.2) (layer "B.Cu") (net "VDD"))
 (segment (start 113.61 76.61) (end 112.46 75.46) (width 0.2) (layer "B.Cu") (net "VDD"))
 (segment (start 115 110.91) (end 115 119.9) (width 0.2) (layer "F.Cu") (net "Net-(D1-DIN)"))
 (segment (start 115 119.9) (end 116.2 121.1) (width 0.2) (layer "F.Cu") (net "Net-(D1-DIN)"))
 (segment (start 119 41.36) (end 119 70.762) (width 0.2) (layer "F.Cu") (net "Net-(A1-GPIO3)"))
 (segment (start 119 70.762) (end 121.158 72.92) (width 0.2) (layer "F.Cu") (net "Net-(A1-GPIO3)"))
 (segment (start 115 37.36) (end 119 41.36) (width 0.2) (layer "F.Cu") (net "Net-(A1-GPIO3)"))
 (segment (start 121.158 73.548) (end 123.15 75.54) (width 0.2) (layer "F.Cu") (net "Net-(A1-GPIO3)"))
 (segment (start 121.158 72.92) (end 121.158 73.548) (width 0.2) (layer "F.Cu") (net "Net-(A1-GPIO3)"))
 (segment (start 121.158 34.92) (end 121.158 35.842) (width 0.2) (layer "F.Cu") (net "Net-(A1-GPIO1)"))
 (segment (start 121.158 34.92) (end 119.668 33.43) (width 0.2) (layer "F.Cu") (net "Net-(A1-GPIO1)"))
 (segment (start 119.668 33.43) (end 113.61 33.43) (width 0.2) (layer "F.Cu") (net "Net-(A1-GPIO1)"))
 (segment (start 121.452 35.842) (end 123.15 37.54) (width 0.2) (layer "F.Cu") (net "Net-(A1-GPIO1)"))
 (segment (start 121.158 35.842) (end 121.452 35.842) (width 0.2) (layer "F.Cu") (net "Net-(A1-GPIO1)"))
 (segment (start 113.61 33.43) (end 112.46 32.28) (width 0.2) (layer "F.Cu") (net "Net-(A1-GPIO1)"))
 (segment (start 140.158 92.548) (end 142.15 94.54) (width 0.2) (layer "F.Cu") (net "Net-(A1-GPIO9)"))
 (segment (start 140.158 91.92) (end 140.158 92.548) (width 0.2) (layer "F.Cu") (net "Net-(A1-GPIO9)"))
 (segment (start 109 48.44) (end 112.46 44.98) (width 0.2) (layer "F.Cu") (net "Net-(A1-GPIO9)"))
 (segment (start 135.238 87) (end 112 87) (width 0.2) (layer "F.Cu") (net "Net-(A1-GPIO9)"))
 (segment (start 112 87) (end 109 84) (width 0.2) (layer "F.Cu") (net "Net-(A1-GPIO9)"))
 (segment (start 140.158 91.92) (end 135.238 87) (width 0.2) (layer "F.Cu") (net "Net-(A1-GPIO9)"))
 (segment (start 109 84) (end 109 48.44) (width 0.2) (layer "F.Cu") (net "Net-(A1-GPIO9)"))
 (segment (start 142.15 56.54) (end 137.538 56.54) (width 0.2) (layer "F.Cu") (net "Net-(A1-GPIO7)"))
 (segment (start 137.538 56.54) (end 126.31 67.768) (width 0.2) (layer "F.Cu") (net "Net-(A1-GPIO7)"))
 (segment (start 116.83 43.83) (end 113.85 43.83) (width 0.2) (layer "F.Cu") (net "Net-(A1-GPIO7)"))
 (segment (start 122.377056 76.88) (end 122.280352 76.88) (width 0.2) (layer "F.Cu") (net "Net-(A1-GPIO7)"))
 (segment (start 123.056295 76.94) (end 122.996295 77) (width 0.2) (layer "F.Cu") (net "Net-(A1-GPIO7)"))
 (segment (start 124.55 75.446295) (end 124.55 76.119899) (width 0.2) (layer "F.Cu") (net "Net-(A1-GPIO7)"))
 (segment (start 124.55 76.119899) (end 123.729899 76.94) (width 0.2) (layer "F.Cu") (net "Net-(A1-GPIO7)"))
 (segment (start 122.280352 76.88) (end 118 72.599648) (width 0.2) (layer "F.Cu") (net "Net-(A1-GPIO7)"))
 (segment (start 126.31 67.768) (end 126.31 73.686295) (width 0.2) (layer "F.Cu") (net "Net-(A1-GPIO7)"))
 (segment (start 123.729899 76.94) (end 123.056295 76.94) (width 0.2) (layer "F.Cu") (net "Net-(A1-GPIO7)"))
 (segment (start 122.996295 77) (end 122.497056 77) (width 0.2) (layer "F.Cu") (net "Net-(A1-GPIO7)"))
 (segment (start 118 45) (end 116.83 43.83) (width 0.2) (layer "F.Cu") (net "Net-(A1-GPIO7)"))
 (segment (start 126.31 73.686295) (end 124.55 75.446295) (width 0.2) (layer "F.Cu") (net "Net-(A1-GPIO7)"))
 (segment (start 113.85 43.83) (end 112.46 42.44) (width 0.2) (layer "F.Cu") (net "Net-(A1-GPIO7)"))
 (segment (start 118 72.599648) (end 118 45) (width 0.2) (layer "F.Cu") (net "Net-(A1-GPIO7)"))
 (segment (start 122.497056 77) (end 122.377056 76.88) (width 0.2) (layer "F.Cu") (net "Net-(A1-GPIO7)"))
 (segment (start 111 84) (end 110 83) (width 0.2) (layer "F.Cu") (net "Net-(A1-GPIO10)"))
 (segment (start 145.31 91.153705) (end 138.156295 84) (width 0.2) (layer "F.Cu") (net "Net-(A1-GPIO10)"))
 (segment (start 110 83) (end 110 49.98) (width 0.2) (layer "F.Cu") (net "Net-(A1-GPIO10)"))
 (segment (start 140.158 99.527225) (end 145.31 94.375225) (width 0.2) (layer "F.Cu") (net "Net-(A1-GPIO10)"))
 (segment (start 145.31 94.375225) (end 145.31 91.153705) (width 0.2) (layer "F.Cu") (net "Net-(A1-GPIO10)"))
 (segment (start 142.15 113.54) (end 140.158 111.548) (width 0.2) (layer "F.Cu") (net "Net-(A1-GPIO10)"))
 (segment (start 140.158 111.548) (end 140.158 99.527225) (width 0.2) (layer "F.Cu") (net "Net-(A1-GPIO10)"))
 (segment (start 138.156295 84) (end 111 84) (width 0.2) (layer "F.Cu") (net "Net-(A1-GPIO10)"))
 (segment (start 110 49.98) (end 112.46 47.52) (width 0.2) (layer "F.Cu") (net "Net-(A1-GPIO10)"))
 (segment (start 117 73) (end 120 76) (width 0.2) (layer "F.Cu") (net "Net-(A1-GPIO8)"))
 (segment (start 138.46 75.54) (end 142.15 75.54) (width 0.2) (layer "F.Cu") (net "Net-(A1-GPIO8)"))
 (segment (start 120 81) (end 121 82) (width 0.2) (layer "F.Cu") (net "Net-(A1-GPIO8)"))
 (segment (start 121 82) (end 132 82) (width 0.2) (layer "F.Cu") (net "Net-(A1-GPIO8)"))
 (segment (start 132 82) (end 138.46 75.54) (width 0.2) (layer "F.Cu") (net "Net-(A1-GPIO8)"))
 (segment (start 120 76) (end 120 81) (width 0.2) (layer "F.Cu") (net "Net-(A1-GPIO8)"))
 (segment (start 117 46.98) (end 117 73) (width 0.2) (layer "F.Cu") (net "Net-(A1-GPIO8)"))
 (segment (start 115 44.98) (end 117 46.98) (width 0.2) (layer "F.Cu") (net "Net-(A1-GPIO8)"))
 (segment (start 113.61 35.97) (end 112.46 34.82) (width 0.2) (layer "F.Cu") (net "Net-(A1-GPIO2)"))
 (segment (start 121.158 54.548) (end 121.158 41.891654) (width 0.2) (layer "F.Cu") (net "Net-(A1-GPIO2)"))
 (segment (start 121.158 41.891654) (end 115.236346 35.97) (width 0.2) (layer "F.Cu") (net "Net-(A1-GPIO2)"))
 (segment (start 123.15 56.54) (end 121.158 54.548) (width 0.2) (layer "F.Cu") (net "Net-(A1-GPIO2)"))
 (segment (start 115.236346 35.97) (end 113.61 35.97) (width 0.2) (layer "F.Cu") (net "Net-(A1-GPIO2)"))
 (segment (start 112.223654 38.51) (end 113.61 38.51) (width 0.2) (layer "F.Cu") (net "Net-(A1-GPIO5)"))
 (segment (start 121.158 111.548) (end 121.158 99.527225) (width 0.2) (layer "F.Cu") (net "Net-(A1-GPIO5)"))
 (segment (start 108 42.733654) (end 112.223654 38.51) (width 0.2) (layer "F.Cu") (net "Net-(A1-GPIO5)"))
 (segment (start 124 88) (end 111 88) (width 0.2) (layer "F.Cu") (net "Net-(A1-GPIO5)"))
 (segment (start 126.31 90.31) (end 124 88) (width 0.2) (layer "F.Cu") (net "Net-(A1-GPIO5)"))
 (segment (start 111 88) (end 108 85) (width 0.2) (layer "F.Cu") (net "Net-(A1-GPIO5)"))
 (segment (start 113.61 38.51) (end 115 39.9) (width 0.2) (layer "F.Cu") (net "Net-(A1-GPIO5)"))
 (segment (start 123.15 113.54) (end 121.158 111.548) (width 0.2) (layer "F.Cu") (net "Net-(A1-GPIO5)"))
 (segment (start 121.158 99.527225) (end 126.31 94.375225) (width 0.2) (layer "F.Cu") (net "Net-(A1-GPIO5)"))
 (segment (start 126.31 94.375225) (end 126.31 90.31) (width 0.2) (layer "F.Cu") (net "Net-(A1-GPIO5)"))
 (segment (start 108 85) (end 108 42.733654) (width 0.2) (layer "F.Cu") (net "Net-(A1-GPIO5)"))
 (segment (start 110 89) (end 107 86) (width 0.2) (layer "F.Cu") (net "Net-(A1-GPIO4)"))
 (segment (start 123.15 94.54) (end 123.15 92.15) (width 0.2) (layer "F.Cu") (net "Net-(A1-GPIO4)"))
 (segment (start 123.15 92.15) (end 122.92 91.92) (width 0.2) (layer "F.Cu") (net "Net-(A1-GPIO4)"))
 (segment (start 117.92 91.92) (end 115 89) (width 0.2) (layer "F.Cu") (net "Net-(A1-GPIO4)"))
 (segment (start 107 42.82) (end 112.46 37.36) (width 0.2) (layer "F.Cu") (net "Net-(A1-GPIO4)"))
 (segment (start 122.92 91.92) (end 117.92 91.92) (width 0.2) (layer "F.Cu") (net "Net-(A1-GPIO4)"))
 (segment (start 115 89) (end 110 89) (width 0.2) (layer "F.Cu") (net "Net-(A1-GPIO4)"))
 (segment (start 107 86) (end 107 42.82) (width 0.2) (layer "F.Cu") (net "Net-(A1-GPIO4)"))
 (segment (start 118 97.75) (end 115 100.75) (width 0.2) (layer "B.Cu") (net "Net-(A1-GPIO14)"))
 (segment (start 115 55.14) (end 118 58.14) (width 0.2) (layer "B.Cu") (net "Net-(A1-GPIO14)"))
 (segment (start 118 58.14) (end 118 97.75) (width 0.2) (layer "B.Cu") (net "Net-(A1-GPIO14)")))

